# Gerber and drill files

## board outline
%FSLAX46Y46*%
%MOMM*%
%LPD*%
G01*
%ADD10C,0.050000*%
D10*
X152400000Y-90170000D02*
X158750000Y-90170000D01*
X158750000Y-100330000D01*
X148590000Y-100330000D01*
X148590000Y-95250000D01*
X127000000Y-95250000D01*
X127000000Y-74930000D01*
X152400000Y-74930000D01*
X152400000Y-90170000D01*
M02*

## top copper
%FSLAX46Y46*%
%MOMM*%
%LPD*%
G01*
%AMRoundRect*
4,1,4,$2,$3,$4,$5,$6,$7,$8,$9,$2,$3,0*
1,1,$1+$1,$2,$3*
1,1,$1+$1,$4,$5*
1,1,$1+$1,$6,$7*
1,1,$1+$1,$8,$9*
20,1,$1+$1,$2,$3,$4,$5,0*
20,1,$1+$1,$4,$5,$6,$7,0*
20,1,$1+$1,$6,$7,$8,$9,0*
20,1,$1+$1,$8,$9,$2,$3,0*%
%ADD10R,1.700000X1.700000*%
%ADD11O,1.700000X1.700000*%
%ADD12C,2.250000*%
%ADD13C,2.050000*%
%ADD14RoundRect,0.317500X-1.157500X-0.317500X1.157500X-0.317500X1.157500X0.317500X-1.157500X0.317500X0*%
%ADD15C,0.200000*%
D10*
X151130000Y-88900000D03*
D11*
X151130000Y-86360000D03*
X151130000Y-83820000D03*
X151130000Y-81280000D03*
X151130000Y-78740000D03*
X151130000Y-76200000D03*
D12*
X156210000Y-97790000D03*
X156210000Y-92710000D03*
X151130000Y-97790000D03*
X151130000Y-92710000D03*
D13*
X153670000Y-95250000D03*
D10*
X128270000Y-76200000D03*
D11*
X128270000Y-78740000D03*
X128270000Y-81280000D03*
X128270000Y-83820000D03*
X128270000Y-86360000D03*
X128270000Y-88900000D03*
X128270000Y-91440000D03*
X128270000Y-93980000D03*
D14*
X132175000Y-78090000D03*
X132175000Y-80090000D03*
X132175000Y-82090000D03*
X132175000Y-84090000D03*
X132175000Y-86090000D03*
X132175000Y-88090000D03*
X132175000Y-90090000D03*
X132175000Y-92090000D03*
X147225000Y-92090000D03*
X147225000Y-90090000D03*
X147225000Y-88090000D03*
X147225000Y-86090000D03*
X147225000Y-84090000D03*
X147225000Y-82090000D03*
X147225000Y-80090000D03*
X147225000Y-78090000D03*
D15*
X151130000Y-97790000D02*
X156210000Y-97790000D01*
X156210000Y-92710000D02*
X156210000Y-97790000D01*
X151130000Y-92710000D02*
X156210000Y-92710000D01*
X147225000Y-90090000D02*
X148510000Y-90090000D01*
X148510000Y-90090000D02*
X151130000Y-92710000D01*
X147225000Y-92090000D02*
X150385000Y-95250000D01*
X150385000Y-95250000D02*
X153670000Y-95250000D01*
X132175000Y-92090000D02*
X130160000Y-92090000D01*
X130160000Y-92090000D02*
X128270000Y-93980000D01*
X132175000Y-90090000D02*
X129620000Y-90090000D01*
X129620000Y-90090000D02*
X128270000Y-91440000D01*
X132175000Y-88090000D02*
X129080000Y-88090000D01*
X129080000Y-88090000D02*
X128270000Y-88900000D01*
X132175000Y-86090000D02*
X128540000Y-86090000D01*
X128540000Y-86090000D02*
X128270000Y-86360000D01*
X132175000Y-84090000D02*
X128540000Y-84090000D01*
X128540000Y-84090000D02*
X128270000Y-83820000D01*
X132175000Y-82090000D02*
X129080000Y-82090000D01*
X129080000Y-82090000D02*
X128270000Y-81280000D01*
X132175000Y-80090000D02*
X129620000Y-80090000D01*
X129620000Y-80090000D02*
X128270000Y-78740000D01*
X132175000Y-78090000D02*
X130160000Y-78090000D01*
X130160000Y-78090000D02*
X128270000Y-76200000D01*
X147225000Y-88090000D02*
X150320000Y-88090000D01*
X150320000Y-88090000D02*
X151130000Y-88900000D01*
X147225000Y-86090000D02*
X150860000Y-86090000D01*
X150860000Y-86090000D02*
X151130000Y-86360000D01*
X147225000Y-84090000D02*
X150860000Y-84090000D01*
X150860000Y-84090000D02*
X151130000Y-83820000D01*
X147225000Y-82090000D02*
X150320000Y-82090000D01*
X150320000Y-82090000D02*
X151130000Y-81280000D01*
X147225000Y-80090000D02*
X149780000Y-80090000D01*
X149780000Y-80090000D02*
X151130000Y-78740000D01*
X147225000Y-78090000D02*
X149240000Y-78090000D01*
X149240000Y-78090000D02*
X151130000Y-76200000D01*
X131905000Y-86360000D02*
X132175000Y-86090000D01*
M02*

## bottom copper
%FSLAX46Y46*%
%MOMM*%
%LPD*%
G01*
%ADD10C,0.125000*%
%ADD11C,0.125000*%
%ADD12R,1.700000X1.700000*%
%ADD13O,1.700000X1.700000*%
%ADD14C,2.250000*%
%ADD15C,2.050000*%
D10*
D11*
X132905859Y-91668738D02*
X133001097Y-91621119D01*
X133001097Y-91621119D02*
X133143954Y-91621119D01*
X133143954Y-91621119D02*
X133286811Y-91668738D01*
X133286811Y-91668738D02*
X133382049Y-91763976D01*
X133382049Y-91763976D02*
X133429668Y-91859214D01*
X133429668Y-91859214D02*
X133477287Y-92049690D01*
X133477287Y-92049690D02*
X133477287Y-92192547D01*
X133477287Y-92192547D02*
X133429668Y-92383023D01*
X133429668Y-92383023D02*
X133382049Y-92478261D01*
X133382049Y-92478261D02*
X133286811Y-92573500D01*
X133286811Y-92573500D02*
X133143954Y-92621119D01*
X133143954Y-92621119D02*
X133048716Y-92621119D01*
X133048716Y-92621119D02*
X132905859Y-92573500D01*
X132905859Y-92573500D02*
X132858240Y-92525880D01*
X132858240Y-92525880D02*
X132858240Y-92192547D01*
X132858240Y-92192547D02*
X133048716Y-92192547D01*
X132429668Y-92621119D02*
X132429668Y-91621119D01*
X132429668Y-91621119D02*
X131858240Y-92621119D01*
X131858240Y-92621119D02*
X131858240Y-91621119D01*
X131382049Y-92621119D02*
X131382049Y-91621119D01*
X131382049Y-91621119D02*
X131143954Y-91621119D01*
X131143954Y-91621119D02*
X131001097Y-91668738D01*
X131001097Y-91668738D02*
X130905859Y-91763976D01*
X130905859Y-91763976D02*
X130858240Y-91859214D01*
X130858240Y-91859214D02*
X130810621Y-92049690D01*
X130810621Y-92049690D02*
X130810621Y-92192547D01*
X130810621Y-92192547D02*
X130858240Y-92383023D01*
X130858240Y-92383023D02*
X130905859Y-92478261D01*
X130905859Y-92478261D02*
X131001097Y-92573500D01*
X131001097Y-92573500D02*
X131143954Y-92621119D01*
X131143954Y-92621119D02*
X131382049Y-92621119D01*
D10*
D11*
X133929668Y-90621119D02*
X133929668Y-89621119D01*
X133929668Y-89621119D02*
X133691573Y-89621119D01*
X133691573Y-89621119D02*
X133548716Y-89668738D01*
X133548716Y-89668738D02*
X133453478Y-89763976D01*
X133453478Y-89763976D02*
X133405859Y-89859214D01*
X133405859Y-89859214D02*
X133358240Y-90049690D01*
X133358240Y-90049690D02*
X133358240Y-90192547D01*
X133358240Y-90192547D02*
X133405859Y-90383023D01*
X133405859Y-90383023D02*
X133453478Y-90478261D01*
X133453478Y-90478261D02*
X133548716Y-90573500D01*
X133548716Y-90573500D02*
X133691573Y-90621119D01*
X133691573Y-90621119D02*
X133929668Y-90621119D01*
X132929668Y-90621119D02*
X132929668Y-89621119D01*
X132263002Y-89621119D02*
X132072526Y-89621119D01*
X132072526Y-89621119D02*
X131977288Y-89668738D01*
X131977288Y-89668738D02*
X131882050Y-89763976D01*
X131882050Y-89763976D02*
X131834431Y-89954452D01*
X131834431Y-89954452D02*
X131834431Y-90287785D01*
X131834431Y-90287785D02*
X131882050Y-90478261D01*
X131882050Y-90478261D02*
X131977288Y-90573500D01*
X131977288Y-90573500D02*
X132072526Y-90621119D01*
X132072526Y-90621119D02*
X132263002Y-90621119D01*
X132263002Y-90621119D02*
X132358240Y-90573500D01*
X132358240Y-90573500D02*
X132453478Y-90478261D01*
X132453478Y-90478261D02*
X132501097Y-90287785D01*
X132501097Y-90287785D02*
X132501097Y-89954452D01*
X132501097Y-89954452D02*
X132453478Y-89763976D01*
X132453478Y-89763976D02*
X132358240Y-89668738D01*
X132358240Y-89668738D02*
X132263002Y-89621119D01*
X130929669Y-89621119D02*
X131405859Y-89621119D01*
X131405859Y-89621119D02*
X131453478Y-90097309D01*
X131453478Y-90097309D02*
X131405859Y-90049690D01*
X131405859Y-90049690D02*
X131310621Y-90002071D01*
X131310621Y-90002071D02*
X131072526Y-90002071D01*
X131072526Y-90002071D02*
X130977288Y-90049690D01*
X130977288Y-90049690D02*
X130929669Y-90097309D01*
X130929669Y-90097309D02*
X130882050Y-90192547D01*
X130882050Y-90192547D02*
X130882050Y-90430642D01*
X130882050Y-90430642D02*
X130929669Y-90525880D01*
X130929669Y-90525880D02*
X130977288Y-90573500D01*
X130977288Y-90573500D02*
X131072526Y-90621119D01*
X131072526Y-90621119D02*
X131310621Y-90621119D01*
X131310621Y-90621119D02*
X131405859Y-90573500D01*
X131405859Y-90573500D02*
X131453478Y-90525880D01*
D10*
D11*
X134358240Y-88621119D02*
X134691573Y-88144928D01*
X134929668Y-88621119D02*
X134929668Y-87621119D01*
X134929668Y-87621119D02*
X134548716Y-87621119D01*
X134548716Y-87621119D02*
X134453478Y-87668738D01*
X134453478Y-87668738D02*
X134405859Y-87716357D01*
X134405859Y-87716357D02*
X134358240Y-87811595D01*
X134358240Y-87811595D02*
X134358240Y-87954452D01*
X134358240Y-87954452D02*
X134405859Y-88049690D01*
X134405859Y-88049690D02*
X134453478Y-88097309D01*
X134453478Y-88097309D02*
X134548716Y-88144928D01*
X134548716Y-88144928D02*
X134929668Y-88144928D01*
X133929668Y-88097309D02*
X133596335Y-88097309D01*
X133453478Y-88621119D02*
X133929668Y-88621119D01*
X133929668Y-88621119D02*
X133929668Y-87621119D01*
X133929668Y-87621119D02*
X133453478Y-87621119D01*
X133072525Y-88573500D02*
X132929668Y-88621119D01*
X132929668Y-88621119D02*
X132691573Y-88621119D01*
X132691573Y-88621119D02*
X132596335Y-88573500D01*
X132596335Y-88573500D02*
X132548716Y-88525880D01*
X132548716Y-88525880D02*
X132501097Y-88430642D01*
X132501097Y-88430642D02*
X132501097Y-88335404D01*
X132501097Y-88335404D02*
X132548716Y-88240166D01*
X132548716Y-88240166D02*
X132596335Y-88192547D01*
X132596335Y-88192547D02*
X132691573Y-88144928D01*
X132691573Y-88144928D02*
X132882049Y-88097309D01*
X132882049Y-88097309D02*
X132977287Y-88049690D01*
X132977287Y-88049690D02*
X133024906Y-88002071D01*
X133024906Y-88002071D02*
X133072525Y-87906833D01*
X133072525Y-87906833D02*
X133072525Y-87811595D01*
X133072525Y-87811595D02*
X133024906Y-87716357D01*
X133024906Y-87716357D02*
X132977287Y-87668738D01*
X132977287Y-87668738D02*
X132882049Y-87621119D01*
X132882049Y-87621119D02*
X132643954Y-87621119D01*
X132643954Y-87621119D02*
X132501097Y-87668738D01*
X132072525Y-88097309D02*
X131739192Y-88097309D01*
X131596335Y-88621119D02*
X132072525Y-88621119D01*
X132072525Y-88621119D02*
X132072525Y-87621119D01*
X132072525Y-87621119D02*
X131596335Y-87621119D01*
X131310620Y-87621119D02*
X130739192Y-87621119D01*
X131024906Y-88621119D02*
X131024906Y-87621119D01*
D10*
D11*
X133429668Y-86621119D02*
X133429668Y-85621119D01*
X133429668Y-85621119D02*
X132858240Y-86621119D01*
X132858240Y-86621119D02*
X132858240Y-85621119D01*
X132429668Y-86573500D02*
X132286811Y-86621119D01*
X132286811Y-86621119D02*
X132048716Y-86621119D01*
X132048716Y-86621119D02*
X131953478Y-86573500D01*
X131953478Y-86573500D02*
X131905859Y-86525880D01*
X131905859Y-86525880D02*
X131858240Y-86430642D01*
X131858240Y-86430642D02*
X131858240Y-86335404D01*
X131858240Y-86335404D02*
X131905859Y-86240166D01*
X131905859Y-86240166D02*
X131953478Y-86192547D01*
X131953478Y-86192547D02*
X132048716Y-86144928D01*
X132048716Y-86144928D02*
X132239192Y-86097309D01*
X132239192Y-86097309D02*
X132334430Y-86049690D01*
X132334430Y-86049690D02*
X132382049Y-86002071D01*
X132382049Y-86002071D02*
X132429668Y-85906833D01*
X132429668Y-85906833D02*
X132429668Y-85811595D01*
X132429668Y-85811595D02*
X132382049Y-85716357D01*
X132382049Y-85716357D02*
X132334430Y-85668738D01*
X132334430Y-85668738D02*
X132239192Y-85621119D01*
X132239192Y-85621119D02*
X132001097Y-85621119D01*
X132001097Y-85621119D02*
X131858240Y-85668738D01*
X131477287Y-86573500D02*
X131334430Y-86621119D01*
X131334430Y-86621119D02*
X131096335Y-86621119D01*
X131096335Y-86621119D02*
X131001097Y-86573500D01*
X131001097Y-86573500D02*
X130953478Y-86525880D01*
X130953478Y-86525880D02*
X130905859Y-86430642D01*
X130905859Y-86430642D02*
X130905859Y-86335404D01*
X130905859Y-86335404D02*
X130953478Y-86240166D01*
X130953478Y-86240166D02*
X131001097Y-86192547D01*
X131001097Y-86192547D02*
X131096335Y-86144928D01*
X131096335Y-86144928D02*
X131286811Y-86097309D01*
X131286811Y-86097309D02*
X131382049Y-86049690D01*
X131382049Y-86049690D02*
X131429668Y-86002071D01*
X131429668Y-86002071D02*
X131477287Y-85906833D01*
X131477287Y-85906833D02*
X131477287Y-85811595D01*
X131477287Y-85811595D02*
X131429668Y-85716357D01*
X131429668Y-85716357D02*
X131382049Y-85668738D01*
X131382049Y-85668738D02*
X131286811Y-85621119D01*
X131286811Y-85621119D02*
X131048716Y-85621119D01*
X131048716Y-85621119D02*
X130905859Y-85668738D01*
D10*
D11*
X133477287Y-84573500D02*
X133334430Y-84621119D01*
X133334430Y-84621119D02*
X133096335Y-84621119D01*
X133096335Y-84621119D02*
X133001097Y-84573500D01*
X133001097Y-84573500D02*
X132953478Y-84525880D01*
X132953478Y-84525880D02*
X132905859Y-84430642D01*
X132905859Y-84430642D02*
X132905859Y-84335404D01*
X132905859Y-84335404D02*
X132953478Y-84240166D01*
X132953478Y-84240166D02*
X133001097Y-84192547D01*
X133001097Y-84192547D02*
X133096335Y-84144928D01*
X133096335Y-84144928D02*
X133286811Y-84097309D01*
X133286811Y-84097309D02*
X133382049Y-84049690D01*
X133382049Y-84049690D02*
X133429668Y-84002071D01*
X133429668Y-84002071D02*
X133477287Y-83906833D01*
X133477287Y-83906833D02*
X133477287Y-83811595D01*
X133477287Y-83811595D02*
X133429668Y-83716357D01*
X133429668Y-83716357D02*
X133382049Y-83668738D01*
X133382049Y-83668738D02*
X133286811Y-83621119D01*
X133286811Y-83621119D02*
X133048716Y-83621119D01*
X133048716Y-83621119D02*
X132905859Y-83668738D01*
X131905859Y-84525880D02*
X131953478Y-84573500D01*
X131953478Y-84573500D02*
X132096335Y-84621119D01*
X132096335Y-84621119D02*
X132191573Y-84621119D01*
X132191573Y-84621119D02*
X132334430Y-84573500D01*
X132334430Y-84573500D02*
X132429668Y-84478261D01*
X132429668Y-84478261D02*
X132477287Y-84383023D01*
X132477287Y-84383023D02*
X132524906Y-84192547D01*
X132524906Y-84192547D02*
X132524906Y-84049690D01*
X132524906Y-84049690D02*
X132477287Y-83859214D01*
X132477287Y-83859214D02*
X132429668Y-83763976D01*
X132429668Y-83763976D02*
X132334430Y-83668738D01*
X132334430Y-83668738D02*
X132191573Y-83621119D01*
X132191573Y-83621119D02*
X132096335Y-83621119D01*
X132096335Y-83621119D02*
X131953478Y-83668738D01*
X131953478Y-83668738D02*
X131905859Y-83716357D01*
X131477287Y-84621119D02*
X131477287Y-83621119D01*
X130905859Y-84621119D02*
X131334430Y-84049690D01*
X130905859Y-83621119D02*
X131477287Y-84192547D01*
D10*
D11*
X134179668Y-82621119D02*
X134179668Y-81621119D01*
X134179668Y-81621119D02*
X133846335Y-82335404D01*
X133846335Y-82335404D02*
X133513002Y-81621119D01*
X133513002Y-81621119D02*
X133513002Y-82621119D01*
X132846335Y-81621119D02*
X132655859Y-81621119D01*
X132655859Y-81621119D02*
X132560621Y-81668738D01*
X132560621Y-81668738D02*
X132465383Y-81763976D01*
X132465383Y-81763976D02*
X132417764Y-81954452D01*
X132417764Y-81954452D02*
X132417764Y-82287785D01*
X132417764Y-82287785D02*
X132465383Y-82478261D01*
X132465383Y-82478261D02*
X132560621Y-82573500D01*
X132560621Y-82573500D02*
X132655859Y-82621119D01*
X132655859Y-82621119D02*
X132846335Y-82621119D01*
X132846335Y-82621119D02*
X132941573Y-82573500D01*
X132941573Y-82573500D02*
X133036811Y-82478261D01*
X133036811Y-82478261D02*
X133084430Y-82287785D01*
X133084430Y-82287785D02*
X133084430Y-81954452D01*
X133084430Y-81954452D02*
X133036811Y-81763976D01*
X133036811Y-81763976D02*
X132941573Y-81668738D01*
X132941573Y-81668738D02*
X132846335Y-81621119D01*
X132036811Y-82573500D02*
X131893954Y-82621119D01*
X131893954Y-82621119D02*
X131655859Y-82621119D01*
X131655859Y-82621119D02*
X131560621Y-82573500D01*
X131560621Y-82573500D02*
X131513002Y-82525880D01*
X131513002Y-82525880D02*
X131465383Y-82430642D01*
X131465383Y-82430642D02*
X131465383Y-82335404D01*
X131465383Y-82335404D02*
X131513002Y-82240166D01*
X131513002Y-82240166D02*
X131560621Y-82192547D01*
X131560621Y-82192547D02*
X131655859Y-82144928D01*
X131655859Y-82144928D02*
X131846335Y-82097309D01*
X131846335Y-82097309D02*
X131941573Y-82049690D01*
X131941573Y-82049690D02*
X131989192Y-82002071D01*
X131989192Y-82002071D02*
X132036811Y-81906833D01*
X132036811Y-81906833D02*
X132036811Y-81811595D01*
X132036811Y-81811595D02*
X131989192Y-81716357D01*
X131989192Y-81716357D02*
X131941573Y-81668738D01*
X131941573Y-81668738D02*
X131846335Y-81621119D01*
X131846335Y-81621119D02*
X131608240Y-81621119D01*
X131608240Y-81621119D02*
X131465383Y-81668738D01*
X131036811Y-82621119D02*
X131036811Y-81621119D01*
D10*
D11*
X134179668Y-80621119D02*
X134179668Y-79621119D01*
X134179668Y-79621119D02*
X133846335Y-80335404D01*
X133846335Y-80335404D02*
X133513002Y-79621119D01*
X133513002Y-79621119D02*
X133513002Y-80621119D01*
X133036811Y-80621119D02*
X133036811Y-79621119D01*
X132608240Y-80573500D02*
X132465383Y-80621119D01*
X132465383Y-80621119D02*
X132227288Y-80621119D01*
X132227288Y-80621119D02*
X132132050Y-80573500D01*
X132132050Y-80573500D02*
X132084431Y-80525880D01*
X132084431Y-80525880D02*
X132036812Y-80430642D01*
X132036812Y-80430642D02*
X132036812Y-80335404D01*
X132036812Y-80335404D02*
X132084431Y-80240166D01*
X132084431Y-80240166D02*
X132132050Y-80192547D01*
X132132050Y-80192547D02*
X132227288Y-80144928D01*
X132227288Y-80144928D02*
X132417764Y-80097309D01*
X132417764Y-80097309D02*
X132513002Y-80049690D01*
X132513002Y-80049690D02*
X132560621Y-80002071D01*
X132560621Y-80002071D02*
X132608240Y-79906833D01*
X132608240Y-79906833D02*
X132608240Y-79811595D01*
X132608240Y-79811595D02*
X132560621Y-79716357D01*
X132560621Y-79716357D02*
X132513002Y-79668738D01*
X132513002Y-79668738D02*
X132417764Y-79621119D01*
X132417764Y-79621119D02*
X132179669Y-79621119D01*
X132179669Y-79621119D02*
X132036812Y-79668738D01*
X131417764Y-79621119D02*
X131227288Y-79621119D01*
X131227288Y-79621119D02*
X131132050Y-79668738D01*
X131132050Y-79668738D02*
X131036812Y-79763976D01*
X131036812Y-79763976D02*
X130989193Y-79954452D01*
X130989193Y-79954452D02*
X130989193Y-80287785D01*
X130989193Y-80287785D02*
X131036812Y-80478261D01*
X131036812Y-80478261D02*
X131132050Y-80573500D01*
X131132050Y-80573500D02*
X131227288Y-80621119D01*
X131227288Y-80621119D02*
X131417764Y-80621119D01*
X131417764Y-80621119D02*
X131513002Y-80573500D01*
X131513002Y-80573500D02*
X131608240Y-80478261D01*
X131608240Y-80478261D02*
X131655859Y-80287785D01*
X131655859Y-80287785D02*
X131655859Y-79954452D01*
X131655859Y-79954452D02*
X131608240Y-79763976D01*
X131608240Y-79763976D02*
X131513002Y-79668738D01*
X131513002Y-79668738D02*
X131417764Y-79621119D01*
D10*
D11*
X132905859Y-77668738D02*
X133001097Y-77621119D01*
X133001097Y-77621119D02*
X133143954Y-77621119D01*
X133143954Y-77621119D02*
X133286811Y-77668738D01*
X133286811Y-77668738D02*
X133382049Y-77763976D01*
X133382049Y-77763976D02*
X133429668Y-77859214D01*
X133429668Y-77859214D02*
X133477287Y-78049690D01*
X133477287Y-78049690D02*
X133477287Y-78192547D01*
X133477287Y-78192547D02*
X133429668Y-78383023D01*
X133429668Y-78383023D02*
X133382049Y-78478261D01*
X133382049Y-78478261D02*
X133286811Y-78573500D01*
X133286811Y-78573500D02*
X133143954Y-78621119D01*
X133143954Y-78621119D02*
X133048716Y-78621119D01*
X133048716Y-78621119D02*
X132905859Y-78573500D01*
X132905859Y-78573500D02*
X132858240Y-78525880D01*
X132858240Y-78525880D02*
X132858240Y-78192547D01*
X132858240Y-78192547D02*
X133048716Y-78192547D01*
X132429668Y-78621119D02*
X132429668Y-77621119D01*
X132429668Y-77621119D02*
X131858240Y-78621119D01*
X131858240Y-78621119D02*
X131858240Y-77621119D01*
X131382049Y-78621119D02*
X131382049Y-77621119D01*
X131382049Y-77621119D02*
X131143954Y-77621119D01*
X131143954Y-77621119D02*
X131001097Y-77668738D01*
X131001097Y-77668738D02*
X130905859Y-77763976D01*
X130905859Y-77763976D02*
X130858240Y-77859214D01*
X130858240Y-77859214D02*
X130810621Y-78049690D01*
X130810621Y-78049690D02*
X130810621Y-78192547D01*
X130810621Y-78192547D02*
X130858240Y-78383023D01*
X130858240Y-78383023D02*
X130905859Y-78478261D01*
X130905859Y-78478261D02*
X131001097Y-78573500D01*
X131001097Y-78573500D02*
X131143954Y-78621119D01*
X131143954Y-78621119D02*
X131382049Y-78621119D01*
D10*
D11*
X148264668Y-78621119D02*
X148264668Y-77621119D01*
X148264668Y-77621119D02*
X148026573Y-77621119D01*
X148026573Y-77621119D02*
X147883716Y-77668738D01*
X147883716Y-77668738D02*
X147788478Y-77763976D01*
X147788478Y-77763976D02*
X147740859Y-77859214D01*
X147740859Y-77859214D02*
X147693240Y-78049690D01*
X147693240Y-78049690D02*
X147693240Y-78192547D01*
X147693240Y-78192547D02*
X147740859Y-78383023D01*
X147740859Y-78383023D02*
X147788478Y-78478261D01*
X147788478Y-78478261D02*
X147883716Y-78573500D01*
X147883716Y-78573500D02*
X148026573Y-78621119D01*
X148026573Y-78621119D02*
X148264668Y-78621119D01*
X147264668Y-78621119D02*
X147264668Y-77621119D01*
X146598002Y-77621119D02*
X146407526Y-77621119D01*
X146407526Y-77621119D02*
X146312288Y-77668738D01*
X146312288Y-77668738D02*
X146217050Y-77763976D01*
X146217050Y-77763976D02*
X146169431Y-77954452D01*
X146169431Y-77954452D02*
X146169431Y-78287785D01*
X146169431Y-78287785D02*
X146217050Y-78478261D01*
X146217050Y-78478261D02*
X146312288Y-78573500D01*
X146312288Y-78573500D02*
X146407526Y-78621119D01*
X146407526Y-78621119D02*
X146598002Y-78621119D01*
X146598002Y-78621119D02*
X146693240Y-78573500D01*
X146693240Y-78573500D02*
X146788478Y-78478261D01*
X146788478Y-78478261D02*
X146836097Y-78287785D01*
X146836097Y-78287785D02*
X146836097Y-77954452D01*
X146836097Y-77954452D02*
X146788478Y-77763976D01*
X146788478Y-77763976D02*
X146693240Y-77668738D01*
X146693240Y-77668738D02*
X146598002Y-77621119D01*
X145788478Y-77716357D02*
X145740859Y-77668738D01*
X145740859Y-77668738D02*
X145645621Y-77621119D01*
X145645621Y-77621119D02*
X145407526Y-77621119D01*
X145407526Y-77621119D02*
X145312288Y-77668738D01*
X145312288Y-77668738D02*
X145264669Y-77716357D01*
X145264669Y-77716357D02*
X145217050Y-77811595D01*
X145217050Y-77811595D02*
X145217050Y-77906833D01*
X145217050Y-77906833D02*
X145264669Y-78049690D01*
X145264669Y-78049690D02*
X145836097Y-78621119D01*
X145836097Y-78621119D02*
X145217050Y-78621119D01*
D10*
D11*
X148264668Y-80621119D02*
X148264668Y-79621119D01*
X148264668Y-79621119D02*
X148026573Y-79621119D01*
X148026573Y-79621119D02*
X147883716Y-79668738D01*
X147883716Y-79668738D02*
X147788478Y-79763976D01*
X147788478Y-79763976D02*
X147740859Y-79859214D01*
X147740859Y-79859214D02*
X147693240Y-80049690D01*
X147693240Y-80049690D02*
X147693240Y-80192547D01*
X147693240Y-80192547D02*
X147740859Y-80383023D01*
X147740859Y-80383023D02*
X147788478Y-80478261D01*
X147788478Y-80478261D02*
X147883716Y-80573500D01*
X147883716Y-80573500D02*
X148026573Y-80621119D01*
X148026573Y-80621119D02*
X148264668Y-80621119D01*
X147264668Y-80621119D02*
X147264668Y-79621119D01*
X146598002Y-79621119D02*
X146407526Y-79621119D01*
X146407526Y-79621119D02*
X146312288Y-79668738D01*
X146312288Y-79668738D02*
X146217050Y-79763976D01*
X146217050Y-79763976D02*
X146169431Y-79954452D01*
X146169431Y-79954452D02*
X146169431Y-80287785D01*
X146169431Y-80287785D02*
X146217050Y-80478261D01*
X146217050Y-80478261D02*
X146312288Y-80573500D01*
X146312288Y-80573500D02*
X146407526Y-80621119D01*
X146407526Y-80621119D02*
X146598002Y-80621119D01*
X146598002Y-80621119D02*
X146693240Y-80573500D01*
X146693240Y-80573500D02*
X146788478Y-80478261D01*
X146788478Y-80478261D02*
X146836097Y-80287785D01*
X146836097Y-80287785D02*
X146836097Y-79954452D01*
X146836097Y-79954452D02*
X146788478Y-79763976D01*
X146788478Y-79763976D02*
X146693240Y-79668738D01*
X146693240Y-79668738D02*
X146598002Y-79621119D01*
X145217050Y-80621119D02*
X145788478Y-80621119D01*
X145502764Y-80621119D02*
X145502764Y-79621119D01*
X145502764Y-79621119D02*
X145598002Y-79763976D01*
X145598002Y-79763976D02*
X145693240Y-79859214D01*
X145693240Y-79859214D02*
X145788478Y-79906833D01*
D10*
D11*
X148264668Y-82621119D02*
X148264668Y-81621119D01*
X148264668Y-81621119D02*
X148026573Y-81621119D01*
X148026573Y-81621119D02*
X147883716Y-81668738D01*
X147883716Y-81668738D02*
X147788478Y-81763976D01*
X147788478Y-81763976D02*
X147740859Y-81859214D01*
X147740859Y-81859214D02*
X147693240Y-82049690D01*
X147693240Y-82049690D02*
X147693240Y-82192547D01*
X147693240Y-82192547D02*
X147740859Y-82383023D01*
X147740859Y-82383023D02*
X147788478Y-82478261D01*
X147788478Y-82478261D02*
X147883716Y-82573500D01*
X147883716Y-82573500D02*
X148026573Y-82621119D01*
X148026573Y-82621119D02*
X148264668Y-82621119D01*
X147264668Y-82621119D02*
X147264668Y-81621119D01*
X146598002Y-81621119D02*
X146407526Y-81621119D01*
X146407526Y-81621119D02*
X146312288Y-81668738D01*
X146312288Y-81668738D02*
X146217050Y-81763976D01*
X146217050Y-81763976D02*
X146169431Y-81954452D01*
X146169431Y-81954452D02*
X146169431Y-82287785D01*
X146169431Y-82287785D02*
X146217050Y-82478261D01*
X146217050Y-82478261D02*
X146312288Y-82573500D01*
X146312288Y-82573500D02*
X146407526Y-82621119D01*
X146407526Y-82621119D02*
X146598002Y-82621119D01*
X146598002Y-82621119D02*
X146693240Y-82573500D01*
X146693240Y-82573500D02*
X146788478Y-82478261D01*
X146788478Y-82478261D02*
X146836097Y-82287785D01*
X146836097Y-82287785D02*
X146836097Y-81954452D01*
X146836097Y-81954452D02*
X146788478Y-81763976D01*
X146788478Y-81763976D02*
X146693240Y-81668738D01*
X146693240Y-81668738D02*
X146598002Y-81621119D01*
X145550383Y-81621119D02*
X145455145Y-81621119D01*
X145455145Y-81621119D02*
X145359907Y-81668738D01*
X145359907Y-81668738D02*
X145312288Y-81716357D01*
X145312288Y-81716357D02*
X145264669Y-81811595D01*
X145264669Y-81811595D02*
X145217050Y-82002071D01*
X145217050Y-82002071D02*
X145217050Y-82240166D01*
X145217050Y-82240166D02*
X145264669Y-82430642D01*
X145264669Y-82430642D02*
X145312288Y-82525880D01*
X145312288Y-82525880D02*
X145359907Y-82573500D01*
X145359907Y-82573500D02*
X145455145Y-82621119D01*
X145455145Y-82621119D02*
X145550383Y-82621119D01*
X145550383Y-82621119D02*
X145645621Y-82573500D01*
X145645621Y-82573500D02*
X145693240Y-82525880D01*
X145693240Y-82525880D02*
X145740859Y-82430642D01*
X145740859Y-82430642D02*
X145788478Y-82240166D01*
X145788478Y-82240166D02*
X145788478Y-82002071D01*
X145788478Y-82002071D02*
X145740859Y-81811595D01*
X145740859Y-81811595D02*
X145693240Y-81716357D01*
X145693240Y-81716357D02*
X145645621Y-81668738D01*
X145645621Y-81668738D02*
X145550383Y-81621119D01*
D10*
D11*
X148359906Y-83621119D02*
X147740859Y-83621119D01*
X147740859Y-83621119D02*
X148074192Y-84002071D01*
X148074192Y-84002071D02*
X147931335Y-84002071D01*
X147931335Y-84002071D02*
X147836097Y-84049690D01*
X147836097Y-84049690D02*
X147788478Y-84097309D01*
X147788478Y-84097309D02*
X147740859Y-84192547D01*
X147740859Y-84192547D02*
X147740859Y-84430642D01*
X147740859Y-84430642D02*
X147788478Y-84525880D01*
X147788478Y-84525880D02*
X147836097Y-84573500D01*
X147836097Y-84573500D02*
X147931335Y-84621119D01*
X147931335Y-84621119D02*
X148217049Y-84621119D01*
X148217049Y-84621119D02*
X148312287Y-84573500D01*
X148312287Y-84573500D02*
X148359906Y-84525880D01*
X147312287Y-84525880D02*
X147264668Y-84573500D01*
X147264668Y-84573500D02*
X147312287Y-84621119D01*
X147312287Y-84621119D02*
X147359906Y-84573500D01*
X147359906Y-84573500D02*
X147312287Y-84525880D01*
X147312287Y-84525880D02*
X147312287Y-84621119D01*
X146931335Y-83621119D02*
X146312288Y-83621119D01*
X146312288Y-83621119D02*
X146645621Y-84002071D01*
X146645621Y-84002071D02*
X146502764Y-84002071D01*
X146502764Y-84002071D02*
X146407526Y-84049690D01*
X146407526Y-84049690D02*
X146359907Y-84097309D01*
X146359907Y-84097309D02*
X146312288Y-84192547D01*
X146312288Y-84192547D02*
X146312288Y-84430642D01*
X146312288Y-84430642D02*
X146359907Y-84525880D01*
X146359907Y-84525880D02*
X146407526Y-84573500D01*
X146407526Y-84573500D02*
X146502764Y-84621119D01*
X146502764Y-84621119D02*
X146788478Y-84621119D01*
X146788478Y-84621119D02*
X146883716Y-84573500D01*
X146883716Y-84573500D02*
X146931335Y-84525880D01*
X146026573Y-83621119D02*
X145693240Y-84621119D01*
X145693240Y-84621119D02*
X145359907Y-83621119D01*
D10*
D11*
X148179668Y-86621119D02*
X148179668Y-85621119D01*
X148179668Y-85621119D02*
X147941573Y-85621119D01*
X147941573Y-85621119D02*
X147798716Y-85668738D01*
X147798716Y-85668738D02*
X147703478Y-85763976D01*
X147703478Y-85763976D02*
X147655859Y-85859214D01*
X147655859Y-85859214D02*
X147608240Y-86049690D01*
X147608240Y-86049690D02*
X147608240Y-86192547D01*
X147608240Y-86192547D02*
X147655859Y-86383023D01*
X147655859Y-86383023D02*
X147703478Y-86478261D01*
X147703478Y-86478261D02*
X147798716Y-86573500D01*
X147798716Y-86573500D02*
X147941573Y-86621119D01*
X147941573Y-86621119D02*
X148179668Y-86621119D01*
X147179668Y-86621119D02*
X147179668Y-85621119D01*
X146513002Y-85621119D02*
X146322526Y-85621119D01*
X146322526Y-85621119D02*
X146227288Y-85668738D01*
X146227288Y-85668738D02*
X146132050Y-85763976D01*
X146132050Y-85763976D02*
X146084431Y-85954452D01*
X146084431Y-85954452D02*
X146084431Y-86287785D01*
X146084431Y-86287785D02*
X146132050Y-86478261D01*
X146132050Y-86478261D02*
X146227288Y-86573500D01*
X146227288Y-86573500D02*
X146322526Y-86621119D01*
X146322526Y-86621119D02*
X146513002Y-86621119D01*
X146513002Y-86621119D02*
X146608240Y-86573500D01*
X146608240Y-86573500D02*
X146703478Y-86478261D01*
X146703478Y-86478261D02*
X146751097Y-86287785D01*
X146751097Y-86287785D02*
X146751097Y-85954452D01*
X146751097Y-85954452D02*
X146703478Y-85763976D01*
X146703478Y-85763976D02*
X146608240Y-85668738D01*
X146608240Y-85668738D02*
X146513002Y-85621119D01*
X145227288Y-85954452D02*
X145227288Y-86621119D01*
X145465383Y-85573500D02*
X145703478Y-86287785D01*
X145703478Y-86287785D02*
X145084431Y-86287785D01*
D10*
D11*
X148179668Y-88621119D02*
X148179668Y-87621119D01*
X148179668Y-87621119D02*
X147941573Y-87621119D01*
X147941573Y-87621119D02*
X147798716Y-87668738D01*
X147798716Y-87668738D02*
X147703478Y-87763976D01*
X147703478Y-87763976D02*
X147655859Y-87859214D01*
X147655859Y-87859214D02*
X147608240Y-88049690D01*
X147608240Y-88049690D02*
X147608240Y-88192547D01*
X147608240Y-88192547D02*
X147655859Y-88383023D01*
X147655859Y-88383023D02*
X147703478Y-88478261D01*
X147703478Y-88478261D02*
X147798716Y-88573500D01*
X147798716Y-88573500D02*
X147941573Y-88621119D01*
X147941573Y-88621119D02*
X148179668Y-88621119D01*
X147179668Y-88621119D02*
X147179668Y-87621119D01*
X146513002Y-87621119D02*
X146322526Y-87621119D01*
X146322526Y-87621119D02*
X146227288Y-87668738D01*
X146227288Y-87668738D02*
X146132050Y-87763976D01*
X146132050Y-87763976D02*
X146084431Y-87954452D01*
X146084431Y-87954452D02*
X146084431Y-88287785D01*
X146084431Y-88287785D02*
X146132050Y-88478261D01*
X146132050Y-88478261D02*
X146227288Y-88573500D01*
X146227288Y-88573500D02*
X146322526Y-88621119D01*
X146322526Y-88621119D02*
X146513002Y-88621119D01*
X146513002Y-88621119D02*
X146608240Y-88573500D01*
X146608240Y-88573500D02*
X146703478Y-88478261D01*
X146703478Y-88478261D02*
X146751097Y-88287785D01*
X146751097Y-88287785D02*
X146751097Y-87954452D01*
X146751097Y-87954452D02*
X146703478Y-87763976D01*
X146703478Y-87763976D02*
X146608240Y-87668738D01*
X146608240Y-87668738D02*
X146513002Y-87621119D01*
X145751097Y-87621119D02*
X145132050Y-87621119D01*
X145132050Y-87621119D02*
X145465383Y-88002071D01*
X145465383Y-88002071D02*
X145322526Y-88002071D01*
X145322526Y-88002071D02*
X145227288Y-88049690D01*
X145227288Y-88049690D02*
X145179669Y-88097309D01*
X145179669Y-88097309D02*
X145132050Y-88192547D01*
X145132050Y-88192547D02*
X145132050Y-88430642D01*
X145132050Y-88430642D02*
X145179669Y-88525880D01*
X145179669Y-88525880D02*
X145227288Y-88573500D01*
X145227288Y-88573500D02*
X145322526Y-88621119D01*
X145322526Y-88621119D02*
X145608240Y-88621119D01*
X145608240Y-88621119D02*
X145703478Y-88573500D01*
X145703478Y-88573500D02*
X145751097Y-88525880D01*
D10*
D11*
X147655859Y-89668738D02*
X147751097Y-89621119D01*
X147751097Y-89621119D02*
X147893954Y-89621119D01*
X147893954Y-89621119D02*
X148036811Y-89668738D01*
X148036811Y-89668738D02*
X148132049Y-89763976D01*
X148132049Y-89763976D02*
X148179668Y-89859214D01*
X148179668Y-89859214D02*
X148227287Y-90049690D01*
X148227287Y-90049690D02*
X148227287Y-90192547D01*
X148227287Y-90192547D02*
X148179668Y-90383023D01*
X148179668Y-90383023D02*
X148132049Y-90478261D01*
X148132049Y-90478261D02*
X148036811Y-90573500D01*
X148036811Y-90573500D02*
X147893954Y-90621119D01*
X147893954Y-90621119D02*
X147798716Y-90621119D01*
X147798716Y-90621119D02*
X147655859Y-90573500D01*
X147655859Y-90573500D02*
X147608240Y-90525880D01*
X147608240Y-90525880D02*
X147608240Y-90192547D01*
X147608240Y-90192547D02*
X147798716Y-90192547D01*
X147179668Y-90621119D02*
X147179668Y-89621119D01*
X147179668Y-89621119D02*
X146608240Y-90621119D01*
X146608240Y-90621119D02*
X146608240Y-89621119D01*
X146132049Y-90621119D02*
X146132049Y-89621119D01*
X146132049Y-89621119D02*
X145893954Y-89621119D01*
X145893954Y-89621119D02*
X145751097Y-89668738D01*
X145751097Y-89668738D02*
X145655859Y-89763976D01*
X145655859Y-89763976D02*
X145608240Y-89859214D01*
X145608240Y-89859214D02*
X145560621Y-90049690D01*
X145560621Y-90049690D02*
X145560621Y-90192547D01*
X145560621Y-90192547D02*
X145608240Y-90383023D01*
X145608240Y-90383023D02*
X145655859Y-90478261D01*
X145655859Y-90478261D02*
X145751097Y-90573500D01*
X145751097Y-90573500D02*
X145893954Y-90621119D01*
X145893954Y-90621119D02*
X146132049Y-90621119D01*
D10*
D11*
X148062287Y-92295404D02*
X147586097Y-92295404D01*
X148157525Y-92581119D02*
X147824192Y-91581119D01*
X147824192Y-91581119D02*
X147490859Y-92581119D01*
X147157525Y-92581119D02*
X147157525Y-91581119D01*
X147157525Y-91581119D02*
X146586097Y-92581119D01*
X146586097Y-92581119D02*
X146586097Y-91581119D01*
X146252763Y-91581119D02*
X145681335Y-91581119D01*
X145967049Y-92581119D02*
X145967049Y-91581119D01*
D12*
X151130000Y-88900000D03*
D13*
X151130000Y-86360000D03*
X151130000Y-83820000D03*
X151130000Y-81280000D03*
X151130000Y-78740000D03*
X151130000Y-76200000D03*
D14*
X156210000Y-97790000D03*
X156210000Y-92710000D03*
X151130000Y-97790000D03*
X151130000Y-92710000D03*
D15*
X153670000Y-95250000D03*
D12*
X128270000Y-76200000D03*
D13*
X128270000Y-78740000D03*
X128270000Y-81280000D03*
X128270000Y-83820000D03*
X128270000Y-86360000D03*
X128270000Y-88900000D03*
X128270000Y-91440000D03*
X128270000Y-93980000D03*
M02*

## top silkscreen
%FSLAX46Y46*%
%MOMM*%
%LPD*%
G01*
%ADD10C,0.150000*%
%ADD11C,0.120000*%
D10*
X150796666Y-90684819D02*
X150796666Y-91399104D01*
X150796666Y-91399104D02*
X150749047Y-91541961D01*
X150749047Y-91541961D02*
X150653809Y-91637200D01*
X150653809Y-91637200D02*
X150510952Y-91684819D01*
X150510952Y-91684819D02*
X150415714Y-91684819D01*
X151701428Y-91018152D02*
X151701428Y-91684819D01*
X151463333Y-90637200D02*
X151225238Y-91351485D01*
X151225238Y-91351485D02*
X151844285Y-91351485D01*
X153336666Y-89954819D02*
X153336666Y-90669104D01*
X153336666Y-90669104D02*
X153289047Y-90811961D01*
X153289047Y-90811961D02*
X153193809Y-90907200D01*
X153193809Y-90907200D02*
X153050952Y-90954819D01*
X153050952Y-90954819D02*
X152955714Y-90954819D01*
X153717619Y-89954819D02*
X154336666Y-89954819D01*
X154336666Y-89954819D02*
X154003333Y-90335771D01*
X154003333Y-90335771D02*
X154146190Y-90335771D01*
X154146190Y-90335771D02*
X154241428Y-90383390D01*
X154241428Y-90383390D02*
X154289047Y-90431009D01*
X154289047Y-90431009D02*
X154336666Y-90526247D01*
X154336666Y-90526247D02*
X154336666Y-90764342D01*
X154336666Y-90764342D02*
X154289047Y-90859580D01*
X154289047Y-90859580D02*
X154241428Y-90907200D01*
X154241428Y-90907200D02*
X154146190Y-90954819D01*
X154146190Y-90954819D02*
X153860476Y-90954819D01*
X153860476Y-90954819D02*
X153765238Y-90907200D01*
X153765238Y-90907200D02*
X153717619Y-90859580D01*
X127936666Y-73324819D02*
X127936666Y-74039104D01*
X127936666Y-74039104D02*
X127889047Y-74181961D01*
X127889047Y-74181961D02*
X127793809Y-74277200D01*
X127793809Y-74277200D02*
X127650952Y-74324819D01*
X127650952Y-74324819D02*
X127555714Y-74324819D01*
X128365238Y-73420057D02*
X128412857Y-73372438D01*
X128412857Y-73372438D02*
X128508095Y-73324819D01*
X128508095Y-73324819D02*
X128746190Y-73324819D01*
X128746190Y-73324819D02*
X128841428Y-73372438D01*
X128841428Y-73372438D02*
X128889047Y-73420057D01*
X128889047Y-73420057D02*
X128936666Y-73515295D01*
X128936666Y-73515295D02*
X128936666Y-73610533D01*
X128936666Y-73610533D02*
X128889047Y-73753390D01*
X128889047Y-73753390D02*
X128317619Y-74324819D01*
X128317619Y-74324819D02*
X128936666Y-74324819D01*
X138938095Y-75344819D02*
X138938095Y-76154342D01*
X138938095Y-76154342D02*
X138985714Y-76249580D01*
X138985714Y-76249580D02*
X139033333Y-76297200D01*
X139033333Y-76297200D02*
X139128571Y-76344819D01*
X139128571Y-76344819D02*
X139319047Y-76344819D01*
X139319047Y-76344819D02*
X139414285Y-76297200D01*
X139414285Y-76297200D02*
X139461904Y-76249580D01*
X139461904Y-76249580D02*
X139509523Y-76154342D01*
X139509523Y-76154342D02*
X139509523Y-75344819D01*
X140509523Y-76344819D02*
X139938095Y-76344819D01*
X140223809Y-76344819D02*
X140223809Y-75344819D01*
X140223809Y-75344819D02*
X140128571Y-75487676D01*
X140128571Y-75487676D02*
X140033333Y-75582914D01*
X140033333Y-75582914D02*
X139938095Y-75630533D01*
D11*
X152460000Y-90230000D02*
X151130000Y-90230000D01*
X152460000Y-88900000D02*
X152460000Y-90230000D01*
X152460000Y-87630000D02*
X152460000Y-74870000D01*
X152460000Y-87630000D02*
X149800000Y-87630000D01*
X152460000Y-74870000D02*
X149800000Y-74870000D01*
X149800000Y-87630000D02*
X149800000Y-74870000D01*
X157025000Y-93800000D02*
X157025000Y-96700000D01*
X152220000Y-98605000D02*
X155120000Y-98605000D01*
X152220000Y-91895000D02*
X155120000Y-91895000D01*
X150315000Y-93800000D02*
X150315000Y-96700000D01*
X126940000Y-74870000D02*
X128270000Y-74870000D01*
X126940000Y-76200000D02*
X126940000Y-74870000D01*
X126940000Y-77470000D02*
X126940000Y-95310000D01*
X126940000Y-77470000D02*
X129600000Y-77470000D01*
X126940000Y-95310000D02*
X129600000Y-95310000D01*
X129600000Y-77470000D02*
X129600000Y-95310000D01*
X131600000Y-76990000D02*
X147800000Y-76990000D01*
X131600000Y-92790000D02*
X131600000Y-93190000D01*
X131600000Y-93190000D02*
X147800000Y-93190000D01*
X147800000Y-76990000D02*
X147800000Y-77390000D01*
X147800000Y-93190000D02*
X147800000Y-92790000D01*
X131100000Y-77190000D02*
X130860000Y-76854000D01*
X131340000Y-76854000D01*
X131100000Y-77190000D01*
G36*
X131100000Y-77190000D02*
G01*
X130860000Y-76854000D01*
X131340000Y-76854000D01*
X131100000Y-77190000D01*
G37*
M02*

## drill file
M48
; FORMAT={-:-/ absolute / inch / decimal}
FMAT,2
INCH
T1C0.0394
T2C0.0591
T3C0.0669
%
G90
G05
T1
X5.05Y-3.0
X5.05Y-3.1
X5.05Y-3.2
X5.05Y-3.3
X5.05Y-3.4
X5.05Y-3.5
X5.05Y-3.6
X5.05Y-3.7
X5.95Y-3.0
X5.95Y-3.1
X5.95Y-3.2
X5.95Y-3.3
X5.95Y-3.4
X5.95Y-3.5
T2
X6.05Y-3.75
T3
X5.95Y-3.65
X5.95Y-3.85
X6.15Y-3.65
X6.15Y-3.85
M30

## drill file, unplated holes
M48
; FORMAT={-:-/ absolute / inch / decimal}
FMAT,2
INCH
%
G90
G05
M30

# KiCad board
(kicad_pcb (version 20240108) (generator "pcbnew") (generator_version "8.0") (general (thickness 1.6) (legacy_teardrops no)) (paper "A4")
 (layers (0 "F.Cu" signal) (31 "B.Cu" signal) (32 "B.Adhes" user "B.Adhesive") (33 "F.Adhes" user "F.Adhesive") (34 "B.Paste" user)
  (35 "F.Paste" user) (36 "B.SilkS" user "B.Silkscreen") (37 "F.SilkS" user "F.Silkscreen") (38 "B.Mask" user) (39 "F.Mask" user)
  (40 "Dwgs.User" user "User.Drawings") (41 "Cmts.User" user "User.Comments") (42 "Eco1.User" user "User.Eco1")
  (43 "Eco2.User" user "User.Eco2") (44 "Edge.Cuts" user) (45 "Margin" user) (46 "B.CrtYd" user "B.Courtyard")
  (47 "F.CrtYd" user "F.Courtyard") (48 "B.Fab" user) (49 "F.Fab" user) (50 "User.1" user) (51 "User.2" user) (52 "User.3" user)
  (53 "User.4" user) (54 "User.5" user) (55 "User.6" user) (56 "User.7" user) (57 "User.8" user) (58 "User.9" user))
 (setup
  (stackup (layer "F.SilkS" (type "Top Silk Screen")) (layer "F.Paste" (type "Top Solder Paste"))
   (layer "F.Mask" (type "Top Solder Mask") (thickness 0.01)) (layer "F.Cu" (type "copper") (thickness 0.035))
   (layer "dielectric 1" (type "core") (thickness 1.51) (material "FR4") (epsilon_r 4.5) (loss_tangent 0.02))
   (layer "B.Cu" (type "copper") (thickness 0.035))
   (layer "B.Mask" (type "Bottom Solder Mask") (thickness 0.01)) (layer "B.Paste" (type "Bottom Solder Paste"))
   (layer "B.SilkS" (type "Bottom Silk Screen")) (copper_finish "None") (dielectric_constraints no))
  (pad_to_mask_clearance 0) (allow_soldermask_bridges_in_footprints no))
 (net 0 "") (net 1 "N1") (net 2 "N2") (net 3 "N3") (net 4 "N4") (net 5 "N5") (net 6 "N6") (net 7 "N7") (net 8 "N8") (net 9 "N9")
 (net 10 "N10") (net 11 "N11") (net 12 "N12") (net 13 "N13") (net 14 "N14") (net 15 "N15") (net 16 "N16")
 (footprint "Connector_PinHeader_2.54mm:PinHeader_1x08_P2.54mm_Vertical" (layer "F.Cu") (at 128.27 76.2)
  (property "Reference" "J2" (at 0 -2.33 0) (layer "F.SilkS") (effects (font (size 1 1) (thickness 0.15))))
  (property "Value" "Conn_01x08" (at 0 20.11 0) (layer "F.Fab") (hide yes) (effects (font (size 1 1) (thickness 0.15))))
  (fp_line (start -1.33 -1.33) (end 0 -1.33) (stroke (width 0.12) (type solid)) (layer "F.SilkS"))
  (fp_line (start -1.33 0) (end -1.33 -1.33) (stroke (width 0.12) (type solid)) (layer "F.SilkS"))
  (fp_line (start -1.33 1.27) (end -1.33 19.11) (stroke (width 0.12) (type solid)) (layer "F.SilkS"))
  (fp_line (start -1.33 1.27) (end 1.33 1.27) (stroke (width 0.12) (type solid)) (layer "F.SilkS"))
  (fp_line (start -1.33 19.11) (end 1.33 19.11) (stroke (width 0.12) (type solid)) (layer "F.SilkS"))
  (fp_line (start 1.33 1.27) (end 1.33 19.11) (stroke (width 0.12) (type solid)) (layer "F.SilkS"))
  (pad "1" thru_hole rect (at 0 0) (size 1.7 1.7) (drill 1) (layers "*.Cu" "*.Mask") (remove_unused_layers no) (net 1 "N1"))
  (pad "2" thru_hole oval (at 0 2.54) (size 1.7 1.7) (drill 1) (layers "*.Cu" "*.Mask") (remove_unused_layers no) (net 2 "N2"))
  (pad "3" thru_hole oval (at 0 5.08) (size 1.7 1.7) (drill 1) (layers "*.Cu" "*.Mask") (remove_unused_layers no) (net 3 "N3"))
  (pad "4" thru_hole oval (at 0 7.62) (size 1.7 1.7) (drill 1) (layers "*.Cu" "*.Mask") (remove_unused_layers no) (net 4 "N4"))
  (pad "5" thru_hole oval (at 0 10.16) (size 1.7 1.7) (drill 1) (layers "*.Cu" "*.Mask") (remove_unused_layers no) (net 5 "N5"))
  (pad "6" thru_hole oval (at 0 12.7) (size 1.7 1.7) (drill 1) (layers "*.Cu" "*.Mask") (remove_unused_layers no) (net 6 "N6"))
  (pad "7" thru_hole oval (at 0 15.24) (size 1.7 1.7) (drill 1) (layers "*.Cu" "*.Mask") (remove_unused_layers no) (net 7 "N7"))
  (pad "8" thru_hole oval (at 0 17.78) (size 1.7 1.7) (drill 1) (layers "*.Cu" "*.Mask") (remove_unused_layers no) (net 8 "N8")))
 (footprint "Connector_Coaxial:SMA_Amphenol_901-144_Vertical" (layer "F.Cu") (at 153.67 95.25)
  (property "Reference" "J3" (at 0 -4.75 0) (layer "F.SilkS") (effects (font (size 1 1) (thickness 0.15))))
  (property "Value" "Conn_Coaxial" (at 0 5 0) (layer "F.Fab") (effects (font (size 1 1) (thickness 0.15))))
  (fp_line (start -3.355 -1.45) (end -3.355 1.45) (stroke (width 0.12) (type solid)) (layer "F.SilkS"))
  (fp_line (start -1.45 -3.355) (end 1.45 -3.355) (stroke (width 0.12) (type solid)) (layer "F.SilkS"))
  (fp_line (start -1.45 3.355) (end 1.45 3.355) (stroke (width 0.12) (type solid)) (layer "F.SilkS"))
  (fp_line (start 3.355 -1.45) (end 3.355 1.45) (stroke (width 0.12) (type solid)) (layer "F.SilkS"))
  (pad "1" thru_hole circle (at 0 0) (size 2.05 2.05) (drill 1.5) (layers "*.Cu" "*.Mask") (remove_unused_layers no) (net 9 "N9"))
  (pad "2" thru_hole circle (at -2.54 -2.54) (size 2.25 2.25) (drill 1.7) (layers "*.Cu" "*.Mask") (remove_unused_layers no) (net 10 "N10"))
  (pad "2" thru_hole circle (at -2.54 2.54) (size 2.25 2.25) (drill 1.7) (layers "*.Cu" "*.Mask") (remove_unused_layers no) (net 10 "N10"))
  (pad "2" thru_hole circle (at 2.54 -2.54) (size 2.25 2.25) (drill 1.7) (layers "*.Cu" "*.Mask") (remove_unused_layers no) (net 10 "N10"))
  (pad "2" thru_hole circle (at 2.54 2.54) (size 2.25 2.25) (drill 1.7) (layers "*.Cu" "*.Mask") (remove_unused_layers no) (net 10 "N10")))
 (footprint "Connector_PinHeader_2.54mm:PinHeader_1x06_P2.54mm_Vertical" (layer "F.Cu") (at 151.13 88.9 180)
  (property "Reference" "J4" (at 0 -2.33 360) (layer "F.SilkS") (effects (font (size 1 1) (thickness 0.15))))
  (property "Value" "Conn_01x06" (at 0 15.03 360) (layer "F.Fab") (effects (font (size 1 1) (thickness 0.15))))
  (fp_line (start 1.33 1.27) (end 1.33 14.03) (stroke (width 0.12) (type solid)) (layer "F.SilkS"))
  (fp_line (start -1.33 14.03) (end 1.33 14.03) (stroke (width 0.12) (type solid)) (layer "F.SilkS"))
  (fp_line (start -1.33 1.27) (end 1.33 1.27) (stroke (width 0.12) (type solid)) (layer "F.SilkS"))
  (fp_line (start -1.33 1.27) (end -1.33 14.03) (stroke (width 0.12) (type solid)) (layer "F.SilkS"))
  (fp_line (start -1.33 0) (end -1.33 -1.33) (stroke (width 0.12) (type solid)) (layer "F.SilkS"))
  (fp_line (start -1.33 -1.33) (end 0 -1.33) (stroke (width 0.12) (type solid)) (layer "F.SilkS"))
  (pad "1" thru_hole rect (at 0 0 180) (size 1.7 1.7) (drill 1) (layers "*.Cu" "*.Mask") (remove_unused_layers no) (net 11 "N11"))
  (pad "2" thru_hole oval (at 0 2.54 180) (size 1.7 1.7) (drill 1) (layers "*.Cu" "*.Mask") (remove_unused_layers no) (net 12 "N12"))
  (pad "3" thru_hole oval (at 0 5.08 180) (size 1.7 1.7) (drill 1) (layers "*.Cu" "*.Mask") (remove_unused_layers no) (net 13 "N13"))
  (pad "4" thru_hole oval (at 0 7.62 180) (size 1.7 1.7) (drill 1) (layers "*.Cu" "*.Mask") (remove_unused_layers no) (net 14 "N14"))
  (pad "5" thru_hole oval (at 0 10.16 180) (size 1.7 1.7) (drill 1) (layers "*.Cu" "*.Mask") (remove_unused_layers no) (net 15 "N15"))
  (pad "6" thru_hole oval (at 0 12.7 180) (size 1.7 1.7) (drill 1) (layers "*.Cu" "*.Mask") (remove_unused_layers no) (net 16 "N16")))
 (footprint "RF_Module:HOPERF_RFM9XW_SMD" (layer "F.Cu") (at 139.7 85.09)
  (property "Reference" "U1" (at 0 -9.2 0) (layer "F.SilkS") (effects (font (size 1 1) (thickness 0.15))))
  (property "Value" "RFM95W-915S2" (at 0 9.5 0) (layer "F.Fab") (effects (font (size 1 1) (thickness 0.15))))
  (fp_line (start -8.1 -8.1) (end 8.1 -8.1) (stroke (width 0.12) (type solid)) (layer "F.SilkS"))
  (fp_line (start -8.1 7.7) (end -8.1 8.1) (stroke (width 0.12) (type solid)) (layer "F.SilkS"))
  (fp_line (start -8.1 8.1) (end 8.1 8.1) (stroke (width 0.12) (type solid)) (layer "F.SilkS"))
  (fp_line (start 8.1 -8.1) (end 8.1 -7.7) (stroke (width 0.12) (type solid)) (layer "F.SilkS"))
  (fp_line (start 8.1 8.1) (end 8.1 7.7) (stroke (width 0.12) (type solid)) (layer "F.SilkS"))
  (fp_poly
   (pts (xy -8.6 -7.9) (xy -8.84 -8.236) (xy -8.36 -8.236) (xy -8.6 -7.9)) (stroke (width 0.12) (type solid)) (fill solid) (layer "F.SilkS"))
  (pad "1" smd roundrect (at -7.525 -7) (size 2.95 1.27) (layers "F.Cu" "F.Paste" "F.Mask") (roundrect_rratio 0.25) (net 1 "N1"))
  (pad "2" smd roundrect (at -7.525 -5) (size 2.95 1.27) (layers "F.Cu" "F.Paste" "F.Mask") (roundrect_rratio 0.25) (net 2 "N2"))
  (pad "3" smd roundrect (at -7.525 -3) (size 2.95 1.27) (layers "F.Cu" "F.Paste" "F.Mask") (roundrect_rratio 0.25) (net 3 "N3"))
  (pad "4" smd roundrect (at -7.525 -1) (size 2.95 1.27) (layers "F.Cu" "F.Paste" "F.Mask") (roundrect_rratio 0.25) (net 4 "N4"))
  (pad "5" smd roundrect (at -7.525 1) (size 2.95 1.27) (layers "F.Cu" "F.Paste" "F.Mask") (roundrect_rratio 0.25) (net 5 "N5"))
  (pad "6" smd roundrect (at -7.525 3) (size 2.95 1.27) (layers "F.Cu" "F.Paste" "F.Mask") (roundrect_rratio 0.25) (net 6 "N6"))
  (pad "7" smd roundrect (at -7.525 5) (size 2.95 1.27) (layers "F.Cu" "F.Paste" "F.Mask") (roundrect_rratio 0.25) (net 7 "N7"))
  (pad "8" smd roundrect (at -7.525 7) (size 2.95 1.27) (layers "F.Cu" "F.Paste" "F.Mask") (roundrect_rratio 0.25) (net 8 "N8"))
  (pad "9" smd roundrect (at 7.525 7) (size 2.95 1.27) (layers "F.Cu" "F.Paste" "F.Mask") (roundrect_rratio 0.25) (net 9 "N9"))
  (pad "10" smd roundrect (at 7.525 5) (size 2.95 1.27) (layers "F.Cu" "F.Paste" "F.Mask") (roundrect_rratio 0.25) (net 10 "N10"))
  (pad "11" smd roundrect (at 7.525 3) (size 2.95 1.27) (layers "F.Cu" "F.Paste" "F.Mask") (roundrect_rratio 0.25) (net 11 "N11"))
  (pad "12" smd roundrect (at 7.525 1) (size 2.95 1.27) (layers "F.Cu" "F.Paste" "F.Mask") (roundrect_rratio 0.25) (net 12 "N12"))
  (pad "13" smd roundrect (at 7.525 -1) (size 2.95 1.27) (layers "F.Cu" "F.Paste" "F.Mask") (roundrect_rratio 0.25) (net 13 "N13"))
  (pad "14" smd roundrect (at 7.525 -3) (size 2.95 1.27) (layers "F.Cu" "F.Paste" "F.Mask") (roundrect_rratio 0.25) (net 14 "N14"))
  (pad "15" smd roundrect (at 7.525 -5) (size 2.95 1.27) (layers "F.Cu" "F.Paste" "F.Mask") (roundrect_rratio 0.25) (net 15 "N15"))
  (pad "16" smd roundrect (at 7.525 -7) (size 2.95 1.27) (layers "F.Cu" "F.Paste" "F.Mask") (roundrect_rratio 0.25) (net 16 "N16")))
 (gr_poly
  (pts (xy 152.4 74.93) (xy 127 74.93) (xy 127 95.25) (xy 148.59 95.25) (xy 148.59 100.33) (xy 158.75 100.33) (xy 158.75 90.17)
   (xy 152.4 90.17))
  (stroke (width 0.05) (type solid)) (fill none) (layer "Edge.Cuts"))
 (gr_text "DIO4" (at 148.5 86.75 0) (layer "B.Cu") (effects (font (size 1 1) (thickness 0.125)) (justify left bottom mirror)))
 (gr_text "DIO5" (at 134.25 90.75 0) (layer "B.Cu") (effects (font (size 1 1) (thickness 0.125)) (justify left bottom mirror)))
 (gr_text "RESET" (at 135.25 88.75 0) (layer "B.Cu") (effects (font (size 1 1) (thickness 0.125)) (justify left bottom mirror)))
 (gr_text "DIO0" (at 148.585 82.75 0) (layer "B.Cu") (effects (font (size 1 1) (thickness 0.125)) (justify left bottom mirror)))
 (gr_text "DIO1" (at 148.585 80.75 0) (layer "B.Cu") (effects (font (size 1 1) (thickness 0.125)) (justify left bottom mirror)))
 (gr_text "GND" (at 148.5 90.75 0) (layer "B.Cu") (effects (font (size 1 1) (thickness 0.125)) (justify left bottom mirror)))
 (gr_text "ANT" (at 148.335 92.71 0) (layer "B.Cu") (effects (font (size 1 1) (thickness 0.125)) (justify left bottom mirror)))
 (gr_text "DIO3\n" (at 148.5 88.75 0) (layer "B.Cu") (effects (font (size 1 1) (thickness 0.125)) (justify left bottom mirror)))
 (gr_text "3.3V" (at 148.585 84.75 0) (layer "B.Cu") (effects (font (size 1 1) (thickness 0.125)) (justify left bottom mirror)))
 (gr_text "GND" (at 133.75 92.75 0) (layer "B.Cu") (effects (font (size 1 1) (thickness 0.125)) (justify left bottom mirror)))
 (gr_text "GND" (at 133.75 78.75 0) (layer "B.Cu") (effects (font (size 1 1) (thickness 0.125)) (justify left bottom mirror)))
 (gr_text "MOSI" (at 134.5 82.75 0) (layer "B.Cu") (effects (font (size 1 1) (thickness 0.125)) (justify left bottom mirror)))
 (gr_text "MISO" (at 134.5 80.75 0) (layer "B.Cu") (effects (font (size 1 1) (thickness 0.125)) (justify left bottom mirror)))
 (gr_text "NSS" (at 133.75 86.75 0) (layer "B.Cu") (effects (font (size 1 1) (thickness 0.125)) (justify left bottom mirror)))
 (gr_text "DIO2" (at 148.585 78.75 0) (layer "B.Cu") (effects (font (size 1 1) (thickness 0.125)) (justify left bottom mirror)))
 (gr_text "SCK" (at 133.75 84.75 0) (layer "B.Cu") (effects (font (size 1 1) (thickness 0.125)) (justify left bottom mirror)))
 (segment (start 132.175 88.09) (end 129.08 88.09) (width 0.2) (layer "F.Cu") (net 6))
 (segment (start 129.08 88.09) (end 128.27 88.9) (width 0.2) (layer "F.Cu") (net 6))
 (segment (start 132.175 78.09) (end 130.16 78.09) (width 0.2) (layer "F.Cu") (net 1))
 (segment (start 130.16 78.09) (end 128.27 76.2) (width 0.2) (layer "F.Cu") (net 1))
 (segment (start 129.62 90.09) (end 128.27 91.44) (width 0.2) (layer "F.Cu") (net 7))
 (segment (start 132.175 90.09) (end 129.62 90.09) (width 0.2) (layer "F.Cu") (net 7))
 (segment (start 130.16 92.09) (end 128.27 93.98) (width 0.2) (layer "F.Cu") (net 8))
 (segment (start 132.175 92.09) (end 130.16 92.09) (width 0.2) (layer "F.Cu") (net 8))
 (segment (start 129.62 80.09) (end 128.27 78.74) (width 0.2) (layer "F.Cu") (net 2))
 (segment (start 132.175 80.09) (end 129.62 80.09) (width 0.2) (layer "F.Cu") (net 2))
 (segment (start 132.175 82.09) (end 129.08 82.09) (width 0.2) (layer "F.Cu") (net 3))
 (segment (start 129.08 82.09) (end 128.27 81.28) (width 0.2) (layer "F.Cu") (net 3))
 (segment (start 132.175 84.09) (end 128.54 84.09) (width 0.2) (layer "F.Cu") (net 4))
 (segment (start 128.54 84.09) (end 128.27 83.82) (width 0.2) (layer "F.Cu") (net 4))
 (segment (start 131.905 86.36) (end 132.175 86.09) (width 0.2) (layer "F.Cu") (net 5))
 (segment (start 132.175 86.09) (end 128.54 86.09) (width 0.2) (layer "F.Cu") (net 5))
 (segment (start 128.54 86.09) (end 128.27 86.36) (width 0.2) (layer "F.Cu") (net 5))
 (segment (start 147.225 92.09) (end 150.385 95.25) (width 0.2) (layer "F.Cu") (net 9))
 (segment (start 150.385 95.25) (end 153.67 95.25) (width 0.2) (layer "F.Cu") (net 9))
 (segment (start 151.13 92.71) (end 156.21 92.71) (width 0.2) (layer "F.Cu") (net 10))
 (segment (start 147.225 90.09) (end 148.51 90.09) (width 0.2) (layer "F.Cu") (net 10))
 (segment (start 148.51 90.09) (end 151.13 92.71) (width 0.2) (layer "F.Cu") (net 10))
 (segment (start 156.21 92.71) (end 156.21 97.79) (width 0.2) (layer "F.Cu") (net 10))
 (segment (start 151.13 97.79) (end 156.21 97.79) (width 0.2) (layer "F.Cu") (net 10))
 (segment (start 150.86 86.09) (end 151.13 86.36) (width 0.2) (layer "F.Cu") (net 12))
 (segment (start 147.225 86.09) (end 150.86 86.09) (width 0.2) (layer "F.Cu") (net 12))
 (segment (start 147.225 78.09) (end 149.24 78.09) (width 0.2) (layer "F.Cu") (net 16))
 (segment (start 149.24 78.09) (end 151.13 76.2) (width 0.2) (layer "F.Cu") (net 16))
 (segment (start 150.32 88.09) (end 151.13 88.9) (width 0.2) (layer "F.Cu") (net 11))
 (segment (start 147.225 88.09) (end 150.32 88.09) (width 0.2) (layer "F.Cu") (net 11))
 (segment (start 150.32 82.09) (end 151.13 81.28) (width 0.2) (layer "F.Cu") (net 14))
 (segment (start 147.225 82.09) (end 150.32 82.09) (width 0.2) (layer "F.Cu") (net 14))
 (segment (start 147.225 84.09) (end 150.86 84.09) (width 0.2) (layer "F.Cu") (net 13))
 (segment (start 150.86 84.09) (end 151.13 83.82) (width 0.2) (layer "F.Cu") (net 13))
 (segment (start 149.78 80.09) (end 151.13 78.74) (width 0.2) (layer "F.Cu") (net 15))
 (segment (start 147.225 80.09) (end 149.78 80.09) (width 0.2) (layer "F.Cu") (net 15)))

